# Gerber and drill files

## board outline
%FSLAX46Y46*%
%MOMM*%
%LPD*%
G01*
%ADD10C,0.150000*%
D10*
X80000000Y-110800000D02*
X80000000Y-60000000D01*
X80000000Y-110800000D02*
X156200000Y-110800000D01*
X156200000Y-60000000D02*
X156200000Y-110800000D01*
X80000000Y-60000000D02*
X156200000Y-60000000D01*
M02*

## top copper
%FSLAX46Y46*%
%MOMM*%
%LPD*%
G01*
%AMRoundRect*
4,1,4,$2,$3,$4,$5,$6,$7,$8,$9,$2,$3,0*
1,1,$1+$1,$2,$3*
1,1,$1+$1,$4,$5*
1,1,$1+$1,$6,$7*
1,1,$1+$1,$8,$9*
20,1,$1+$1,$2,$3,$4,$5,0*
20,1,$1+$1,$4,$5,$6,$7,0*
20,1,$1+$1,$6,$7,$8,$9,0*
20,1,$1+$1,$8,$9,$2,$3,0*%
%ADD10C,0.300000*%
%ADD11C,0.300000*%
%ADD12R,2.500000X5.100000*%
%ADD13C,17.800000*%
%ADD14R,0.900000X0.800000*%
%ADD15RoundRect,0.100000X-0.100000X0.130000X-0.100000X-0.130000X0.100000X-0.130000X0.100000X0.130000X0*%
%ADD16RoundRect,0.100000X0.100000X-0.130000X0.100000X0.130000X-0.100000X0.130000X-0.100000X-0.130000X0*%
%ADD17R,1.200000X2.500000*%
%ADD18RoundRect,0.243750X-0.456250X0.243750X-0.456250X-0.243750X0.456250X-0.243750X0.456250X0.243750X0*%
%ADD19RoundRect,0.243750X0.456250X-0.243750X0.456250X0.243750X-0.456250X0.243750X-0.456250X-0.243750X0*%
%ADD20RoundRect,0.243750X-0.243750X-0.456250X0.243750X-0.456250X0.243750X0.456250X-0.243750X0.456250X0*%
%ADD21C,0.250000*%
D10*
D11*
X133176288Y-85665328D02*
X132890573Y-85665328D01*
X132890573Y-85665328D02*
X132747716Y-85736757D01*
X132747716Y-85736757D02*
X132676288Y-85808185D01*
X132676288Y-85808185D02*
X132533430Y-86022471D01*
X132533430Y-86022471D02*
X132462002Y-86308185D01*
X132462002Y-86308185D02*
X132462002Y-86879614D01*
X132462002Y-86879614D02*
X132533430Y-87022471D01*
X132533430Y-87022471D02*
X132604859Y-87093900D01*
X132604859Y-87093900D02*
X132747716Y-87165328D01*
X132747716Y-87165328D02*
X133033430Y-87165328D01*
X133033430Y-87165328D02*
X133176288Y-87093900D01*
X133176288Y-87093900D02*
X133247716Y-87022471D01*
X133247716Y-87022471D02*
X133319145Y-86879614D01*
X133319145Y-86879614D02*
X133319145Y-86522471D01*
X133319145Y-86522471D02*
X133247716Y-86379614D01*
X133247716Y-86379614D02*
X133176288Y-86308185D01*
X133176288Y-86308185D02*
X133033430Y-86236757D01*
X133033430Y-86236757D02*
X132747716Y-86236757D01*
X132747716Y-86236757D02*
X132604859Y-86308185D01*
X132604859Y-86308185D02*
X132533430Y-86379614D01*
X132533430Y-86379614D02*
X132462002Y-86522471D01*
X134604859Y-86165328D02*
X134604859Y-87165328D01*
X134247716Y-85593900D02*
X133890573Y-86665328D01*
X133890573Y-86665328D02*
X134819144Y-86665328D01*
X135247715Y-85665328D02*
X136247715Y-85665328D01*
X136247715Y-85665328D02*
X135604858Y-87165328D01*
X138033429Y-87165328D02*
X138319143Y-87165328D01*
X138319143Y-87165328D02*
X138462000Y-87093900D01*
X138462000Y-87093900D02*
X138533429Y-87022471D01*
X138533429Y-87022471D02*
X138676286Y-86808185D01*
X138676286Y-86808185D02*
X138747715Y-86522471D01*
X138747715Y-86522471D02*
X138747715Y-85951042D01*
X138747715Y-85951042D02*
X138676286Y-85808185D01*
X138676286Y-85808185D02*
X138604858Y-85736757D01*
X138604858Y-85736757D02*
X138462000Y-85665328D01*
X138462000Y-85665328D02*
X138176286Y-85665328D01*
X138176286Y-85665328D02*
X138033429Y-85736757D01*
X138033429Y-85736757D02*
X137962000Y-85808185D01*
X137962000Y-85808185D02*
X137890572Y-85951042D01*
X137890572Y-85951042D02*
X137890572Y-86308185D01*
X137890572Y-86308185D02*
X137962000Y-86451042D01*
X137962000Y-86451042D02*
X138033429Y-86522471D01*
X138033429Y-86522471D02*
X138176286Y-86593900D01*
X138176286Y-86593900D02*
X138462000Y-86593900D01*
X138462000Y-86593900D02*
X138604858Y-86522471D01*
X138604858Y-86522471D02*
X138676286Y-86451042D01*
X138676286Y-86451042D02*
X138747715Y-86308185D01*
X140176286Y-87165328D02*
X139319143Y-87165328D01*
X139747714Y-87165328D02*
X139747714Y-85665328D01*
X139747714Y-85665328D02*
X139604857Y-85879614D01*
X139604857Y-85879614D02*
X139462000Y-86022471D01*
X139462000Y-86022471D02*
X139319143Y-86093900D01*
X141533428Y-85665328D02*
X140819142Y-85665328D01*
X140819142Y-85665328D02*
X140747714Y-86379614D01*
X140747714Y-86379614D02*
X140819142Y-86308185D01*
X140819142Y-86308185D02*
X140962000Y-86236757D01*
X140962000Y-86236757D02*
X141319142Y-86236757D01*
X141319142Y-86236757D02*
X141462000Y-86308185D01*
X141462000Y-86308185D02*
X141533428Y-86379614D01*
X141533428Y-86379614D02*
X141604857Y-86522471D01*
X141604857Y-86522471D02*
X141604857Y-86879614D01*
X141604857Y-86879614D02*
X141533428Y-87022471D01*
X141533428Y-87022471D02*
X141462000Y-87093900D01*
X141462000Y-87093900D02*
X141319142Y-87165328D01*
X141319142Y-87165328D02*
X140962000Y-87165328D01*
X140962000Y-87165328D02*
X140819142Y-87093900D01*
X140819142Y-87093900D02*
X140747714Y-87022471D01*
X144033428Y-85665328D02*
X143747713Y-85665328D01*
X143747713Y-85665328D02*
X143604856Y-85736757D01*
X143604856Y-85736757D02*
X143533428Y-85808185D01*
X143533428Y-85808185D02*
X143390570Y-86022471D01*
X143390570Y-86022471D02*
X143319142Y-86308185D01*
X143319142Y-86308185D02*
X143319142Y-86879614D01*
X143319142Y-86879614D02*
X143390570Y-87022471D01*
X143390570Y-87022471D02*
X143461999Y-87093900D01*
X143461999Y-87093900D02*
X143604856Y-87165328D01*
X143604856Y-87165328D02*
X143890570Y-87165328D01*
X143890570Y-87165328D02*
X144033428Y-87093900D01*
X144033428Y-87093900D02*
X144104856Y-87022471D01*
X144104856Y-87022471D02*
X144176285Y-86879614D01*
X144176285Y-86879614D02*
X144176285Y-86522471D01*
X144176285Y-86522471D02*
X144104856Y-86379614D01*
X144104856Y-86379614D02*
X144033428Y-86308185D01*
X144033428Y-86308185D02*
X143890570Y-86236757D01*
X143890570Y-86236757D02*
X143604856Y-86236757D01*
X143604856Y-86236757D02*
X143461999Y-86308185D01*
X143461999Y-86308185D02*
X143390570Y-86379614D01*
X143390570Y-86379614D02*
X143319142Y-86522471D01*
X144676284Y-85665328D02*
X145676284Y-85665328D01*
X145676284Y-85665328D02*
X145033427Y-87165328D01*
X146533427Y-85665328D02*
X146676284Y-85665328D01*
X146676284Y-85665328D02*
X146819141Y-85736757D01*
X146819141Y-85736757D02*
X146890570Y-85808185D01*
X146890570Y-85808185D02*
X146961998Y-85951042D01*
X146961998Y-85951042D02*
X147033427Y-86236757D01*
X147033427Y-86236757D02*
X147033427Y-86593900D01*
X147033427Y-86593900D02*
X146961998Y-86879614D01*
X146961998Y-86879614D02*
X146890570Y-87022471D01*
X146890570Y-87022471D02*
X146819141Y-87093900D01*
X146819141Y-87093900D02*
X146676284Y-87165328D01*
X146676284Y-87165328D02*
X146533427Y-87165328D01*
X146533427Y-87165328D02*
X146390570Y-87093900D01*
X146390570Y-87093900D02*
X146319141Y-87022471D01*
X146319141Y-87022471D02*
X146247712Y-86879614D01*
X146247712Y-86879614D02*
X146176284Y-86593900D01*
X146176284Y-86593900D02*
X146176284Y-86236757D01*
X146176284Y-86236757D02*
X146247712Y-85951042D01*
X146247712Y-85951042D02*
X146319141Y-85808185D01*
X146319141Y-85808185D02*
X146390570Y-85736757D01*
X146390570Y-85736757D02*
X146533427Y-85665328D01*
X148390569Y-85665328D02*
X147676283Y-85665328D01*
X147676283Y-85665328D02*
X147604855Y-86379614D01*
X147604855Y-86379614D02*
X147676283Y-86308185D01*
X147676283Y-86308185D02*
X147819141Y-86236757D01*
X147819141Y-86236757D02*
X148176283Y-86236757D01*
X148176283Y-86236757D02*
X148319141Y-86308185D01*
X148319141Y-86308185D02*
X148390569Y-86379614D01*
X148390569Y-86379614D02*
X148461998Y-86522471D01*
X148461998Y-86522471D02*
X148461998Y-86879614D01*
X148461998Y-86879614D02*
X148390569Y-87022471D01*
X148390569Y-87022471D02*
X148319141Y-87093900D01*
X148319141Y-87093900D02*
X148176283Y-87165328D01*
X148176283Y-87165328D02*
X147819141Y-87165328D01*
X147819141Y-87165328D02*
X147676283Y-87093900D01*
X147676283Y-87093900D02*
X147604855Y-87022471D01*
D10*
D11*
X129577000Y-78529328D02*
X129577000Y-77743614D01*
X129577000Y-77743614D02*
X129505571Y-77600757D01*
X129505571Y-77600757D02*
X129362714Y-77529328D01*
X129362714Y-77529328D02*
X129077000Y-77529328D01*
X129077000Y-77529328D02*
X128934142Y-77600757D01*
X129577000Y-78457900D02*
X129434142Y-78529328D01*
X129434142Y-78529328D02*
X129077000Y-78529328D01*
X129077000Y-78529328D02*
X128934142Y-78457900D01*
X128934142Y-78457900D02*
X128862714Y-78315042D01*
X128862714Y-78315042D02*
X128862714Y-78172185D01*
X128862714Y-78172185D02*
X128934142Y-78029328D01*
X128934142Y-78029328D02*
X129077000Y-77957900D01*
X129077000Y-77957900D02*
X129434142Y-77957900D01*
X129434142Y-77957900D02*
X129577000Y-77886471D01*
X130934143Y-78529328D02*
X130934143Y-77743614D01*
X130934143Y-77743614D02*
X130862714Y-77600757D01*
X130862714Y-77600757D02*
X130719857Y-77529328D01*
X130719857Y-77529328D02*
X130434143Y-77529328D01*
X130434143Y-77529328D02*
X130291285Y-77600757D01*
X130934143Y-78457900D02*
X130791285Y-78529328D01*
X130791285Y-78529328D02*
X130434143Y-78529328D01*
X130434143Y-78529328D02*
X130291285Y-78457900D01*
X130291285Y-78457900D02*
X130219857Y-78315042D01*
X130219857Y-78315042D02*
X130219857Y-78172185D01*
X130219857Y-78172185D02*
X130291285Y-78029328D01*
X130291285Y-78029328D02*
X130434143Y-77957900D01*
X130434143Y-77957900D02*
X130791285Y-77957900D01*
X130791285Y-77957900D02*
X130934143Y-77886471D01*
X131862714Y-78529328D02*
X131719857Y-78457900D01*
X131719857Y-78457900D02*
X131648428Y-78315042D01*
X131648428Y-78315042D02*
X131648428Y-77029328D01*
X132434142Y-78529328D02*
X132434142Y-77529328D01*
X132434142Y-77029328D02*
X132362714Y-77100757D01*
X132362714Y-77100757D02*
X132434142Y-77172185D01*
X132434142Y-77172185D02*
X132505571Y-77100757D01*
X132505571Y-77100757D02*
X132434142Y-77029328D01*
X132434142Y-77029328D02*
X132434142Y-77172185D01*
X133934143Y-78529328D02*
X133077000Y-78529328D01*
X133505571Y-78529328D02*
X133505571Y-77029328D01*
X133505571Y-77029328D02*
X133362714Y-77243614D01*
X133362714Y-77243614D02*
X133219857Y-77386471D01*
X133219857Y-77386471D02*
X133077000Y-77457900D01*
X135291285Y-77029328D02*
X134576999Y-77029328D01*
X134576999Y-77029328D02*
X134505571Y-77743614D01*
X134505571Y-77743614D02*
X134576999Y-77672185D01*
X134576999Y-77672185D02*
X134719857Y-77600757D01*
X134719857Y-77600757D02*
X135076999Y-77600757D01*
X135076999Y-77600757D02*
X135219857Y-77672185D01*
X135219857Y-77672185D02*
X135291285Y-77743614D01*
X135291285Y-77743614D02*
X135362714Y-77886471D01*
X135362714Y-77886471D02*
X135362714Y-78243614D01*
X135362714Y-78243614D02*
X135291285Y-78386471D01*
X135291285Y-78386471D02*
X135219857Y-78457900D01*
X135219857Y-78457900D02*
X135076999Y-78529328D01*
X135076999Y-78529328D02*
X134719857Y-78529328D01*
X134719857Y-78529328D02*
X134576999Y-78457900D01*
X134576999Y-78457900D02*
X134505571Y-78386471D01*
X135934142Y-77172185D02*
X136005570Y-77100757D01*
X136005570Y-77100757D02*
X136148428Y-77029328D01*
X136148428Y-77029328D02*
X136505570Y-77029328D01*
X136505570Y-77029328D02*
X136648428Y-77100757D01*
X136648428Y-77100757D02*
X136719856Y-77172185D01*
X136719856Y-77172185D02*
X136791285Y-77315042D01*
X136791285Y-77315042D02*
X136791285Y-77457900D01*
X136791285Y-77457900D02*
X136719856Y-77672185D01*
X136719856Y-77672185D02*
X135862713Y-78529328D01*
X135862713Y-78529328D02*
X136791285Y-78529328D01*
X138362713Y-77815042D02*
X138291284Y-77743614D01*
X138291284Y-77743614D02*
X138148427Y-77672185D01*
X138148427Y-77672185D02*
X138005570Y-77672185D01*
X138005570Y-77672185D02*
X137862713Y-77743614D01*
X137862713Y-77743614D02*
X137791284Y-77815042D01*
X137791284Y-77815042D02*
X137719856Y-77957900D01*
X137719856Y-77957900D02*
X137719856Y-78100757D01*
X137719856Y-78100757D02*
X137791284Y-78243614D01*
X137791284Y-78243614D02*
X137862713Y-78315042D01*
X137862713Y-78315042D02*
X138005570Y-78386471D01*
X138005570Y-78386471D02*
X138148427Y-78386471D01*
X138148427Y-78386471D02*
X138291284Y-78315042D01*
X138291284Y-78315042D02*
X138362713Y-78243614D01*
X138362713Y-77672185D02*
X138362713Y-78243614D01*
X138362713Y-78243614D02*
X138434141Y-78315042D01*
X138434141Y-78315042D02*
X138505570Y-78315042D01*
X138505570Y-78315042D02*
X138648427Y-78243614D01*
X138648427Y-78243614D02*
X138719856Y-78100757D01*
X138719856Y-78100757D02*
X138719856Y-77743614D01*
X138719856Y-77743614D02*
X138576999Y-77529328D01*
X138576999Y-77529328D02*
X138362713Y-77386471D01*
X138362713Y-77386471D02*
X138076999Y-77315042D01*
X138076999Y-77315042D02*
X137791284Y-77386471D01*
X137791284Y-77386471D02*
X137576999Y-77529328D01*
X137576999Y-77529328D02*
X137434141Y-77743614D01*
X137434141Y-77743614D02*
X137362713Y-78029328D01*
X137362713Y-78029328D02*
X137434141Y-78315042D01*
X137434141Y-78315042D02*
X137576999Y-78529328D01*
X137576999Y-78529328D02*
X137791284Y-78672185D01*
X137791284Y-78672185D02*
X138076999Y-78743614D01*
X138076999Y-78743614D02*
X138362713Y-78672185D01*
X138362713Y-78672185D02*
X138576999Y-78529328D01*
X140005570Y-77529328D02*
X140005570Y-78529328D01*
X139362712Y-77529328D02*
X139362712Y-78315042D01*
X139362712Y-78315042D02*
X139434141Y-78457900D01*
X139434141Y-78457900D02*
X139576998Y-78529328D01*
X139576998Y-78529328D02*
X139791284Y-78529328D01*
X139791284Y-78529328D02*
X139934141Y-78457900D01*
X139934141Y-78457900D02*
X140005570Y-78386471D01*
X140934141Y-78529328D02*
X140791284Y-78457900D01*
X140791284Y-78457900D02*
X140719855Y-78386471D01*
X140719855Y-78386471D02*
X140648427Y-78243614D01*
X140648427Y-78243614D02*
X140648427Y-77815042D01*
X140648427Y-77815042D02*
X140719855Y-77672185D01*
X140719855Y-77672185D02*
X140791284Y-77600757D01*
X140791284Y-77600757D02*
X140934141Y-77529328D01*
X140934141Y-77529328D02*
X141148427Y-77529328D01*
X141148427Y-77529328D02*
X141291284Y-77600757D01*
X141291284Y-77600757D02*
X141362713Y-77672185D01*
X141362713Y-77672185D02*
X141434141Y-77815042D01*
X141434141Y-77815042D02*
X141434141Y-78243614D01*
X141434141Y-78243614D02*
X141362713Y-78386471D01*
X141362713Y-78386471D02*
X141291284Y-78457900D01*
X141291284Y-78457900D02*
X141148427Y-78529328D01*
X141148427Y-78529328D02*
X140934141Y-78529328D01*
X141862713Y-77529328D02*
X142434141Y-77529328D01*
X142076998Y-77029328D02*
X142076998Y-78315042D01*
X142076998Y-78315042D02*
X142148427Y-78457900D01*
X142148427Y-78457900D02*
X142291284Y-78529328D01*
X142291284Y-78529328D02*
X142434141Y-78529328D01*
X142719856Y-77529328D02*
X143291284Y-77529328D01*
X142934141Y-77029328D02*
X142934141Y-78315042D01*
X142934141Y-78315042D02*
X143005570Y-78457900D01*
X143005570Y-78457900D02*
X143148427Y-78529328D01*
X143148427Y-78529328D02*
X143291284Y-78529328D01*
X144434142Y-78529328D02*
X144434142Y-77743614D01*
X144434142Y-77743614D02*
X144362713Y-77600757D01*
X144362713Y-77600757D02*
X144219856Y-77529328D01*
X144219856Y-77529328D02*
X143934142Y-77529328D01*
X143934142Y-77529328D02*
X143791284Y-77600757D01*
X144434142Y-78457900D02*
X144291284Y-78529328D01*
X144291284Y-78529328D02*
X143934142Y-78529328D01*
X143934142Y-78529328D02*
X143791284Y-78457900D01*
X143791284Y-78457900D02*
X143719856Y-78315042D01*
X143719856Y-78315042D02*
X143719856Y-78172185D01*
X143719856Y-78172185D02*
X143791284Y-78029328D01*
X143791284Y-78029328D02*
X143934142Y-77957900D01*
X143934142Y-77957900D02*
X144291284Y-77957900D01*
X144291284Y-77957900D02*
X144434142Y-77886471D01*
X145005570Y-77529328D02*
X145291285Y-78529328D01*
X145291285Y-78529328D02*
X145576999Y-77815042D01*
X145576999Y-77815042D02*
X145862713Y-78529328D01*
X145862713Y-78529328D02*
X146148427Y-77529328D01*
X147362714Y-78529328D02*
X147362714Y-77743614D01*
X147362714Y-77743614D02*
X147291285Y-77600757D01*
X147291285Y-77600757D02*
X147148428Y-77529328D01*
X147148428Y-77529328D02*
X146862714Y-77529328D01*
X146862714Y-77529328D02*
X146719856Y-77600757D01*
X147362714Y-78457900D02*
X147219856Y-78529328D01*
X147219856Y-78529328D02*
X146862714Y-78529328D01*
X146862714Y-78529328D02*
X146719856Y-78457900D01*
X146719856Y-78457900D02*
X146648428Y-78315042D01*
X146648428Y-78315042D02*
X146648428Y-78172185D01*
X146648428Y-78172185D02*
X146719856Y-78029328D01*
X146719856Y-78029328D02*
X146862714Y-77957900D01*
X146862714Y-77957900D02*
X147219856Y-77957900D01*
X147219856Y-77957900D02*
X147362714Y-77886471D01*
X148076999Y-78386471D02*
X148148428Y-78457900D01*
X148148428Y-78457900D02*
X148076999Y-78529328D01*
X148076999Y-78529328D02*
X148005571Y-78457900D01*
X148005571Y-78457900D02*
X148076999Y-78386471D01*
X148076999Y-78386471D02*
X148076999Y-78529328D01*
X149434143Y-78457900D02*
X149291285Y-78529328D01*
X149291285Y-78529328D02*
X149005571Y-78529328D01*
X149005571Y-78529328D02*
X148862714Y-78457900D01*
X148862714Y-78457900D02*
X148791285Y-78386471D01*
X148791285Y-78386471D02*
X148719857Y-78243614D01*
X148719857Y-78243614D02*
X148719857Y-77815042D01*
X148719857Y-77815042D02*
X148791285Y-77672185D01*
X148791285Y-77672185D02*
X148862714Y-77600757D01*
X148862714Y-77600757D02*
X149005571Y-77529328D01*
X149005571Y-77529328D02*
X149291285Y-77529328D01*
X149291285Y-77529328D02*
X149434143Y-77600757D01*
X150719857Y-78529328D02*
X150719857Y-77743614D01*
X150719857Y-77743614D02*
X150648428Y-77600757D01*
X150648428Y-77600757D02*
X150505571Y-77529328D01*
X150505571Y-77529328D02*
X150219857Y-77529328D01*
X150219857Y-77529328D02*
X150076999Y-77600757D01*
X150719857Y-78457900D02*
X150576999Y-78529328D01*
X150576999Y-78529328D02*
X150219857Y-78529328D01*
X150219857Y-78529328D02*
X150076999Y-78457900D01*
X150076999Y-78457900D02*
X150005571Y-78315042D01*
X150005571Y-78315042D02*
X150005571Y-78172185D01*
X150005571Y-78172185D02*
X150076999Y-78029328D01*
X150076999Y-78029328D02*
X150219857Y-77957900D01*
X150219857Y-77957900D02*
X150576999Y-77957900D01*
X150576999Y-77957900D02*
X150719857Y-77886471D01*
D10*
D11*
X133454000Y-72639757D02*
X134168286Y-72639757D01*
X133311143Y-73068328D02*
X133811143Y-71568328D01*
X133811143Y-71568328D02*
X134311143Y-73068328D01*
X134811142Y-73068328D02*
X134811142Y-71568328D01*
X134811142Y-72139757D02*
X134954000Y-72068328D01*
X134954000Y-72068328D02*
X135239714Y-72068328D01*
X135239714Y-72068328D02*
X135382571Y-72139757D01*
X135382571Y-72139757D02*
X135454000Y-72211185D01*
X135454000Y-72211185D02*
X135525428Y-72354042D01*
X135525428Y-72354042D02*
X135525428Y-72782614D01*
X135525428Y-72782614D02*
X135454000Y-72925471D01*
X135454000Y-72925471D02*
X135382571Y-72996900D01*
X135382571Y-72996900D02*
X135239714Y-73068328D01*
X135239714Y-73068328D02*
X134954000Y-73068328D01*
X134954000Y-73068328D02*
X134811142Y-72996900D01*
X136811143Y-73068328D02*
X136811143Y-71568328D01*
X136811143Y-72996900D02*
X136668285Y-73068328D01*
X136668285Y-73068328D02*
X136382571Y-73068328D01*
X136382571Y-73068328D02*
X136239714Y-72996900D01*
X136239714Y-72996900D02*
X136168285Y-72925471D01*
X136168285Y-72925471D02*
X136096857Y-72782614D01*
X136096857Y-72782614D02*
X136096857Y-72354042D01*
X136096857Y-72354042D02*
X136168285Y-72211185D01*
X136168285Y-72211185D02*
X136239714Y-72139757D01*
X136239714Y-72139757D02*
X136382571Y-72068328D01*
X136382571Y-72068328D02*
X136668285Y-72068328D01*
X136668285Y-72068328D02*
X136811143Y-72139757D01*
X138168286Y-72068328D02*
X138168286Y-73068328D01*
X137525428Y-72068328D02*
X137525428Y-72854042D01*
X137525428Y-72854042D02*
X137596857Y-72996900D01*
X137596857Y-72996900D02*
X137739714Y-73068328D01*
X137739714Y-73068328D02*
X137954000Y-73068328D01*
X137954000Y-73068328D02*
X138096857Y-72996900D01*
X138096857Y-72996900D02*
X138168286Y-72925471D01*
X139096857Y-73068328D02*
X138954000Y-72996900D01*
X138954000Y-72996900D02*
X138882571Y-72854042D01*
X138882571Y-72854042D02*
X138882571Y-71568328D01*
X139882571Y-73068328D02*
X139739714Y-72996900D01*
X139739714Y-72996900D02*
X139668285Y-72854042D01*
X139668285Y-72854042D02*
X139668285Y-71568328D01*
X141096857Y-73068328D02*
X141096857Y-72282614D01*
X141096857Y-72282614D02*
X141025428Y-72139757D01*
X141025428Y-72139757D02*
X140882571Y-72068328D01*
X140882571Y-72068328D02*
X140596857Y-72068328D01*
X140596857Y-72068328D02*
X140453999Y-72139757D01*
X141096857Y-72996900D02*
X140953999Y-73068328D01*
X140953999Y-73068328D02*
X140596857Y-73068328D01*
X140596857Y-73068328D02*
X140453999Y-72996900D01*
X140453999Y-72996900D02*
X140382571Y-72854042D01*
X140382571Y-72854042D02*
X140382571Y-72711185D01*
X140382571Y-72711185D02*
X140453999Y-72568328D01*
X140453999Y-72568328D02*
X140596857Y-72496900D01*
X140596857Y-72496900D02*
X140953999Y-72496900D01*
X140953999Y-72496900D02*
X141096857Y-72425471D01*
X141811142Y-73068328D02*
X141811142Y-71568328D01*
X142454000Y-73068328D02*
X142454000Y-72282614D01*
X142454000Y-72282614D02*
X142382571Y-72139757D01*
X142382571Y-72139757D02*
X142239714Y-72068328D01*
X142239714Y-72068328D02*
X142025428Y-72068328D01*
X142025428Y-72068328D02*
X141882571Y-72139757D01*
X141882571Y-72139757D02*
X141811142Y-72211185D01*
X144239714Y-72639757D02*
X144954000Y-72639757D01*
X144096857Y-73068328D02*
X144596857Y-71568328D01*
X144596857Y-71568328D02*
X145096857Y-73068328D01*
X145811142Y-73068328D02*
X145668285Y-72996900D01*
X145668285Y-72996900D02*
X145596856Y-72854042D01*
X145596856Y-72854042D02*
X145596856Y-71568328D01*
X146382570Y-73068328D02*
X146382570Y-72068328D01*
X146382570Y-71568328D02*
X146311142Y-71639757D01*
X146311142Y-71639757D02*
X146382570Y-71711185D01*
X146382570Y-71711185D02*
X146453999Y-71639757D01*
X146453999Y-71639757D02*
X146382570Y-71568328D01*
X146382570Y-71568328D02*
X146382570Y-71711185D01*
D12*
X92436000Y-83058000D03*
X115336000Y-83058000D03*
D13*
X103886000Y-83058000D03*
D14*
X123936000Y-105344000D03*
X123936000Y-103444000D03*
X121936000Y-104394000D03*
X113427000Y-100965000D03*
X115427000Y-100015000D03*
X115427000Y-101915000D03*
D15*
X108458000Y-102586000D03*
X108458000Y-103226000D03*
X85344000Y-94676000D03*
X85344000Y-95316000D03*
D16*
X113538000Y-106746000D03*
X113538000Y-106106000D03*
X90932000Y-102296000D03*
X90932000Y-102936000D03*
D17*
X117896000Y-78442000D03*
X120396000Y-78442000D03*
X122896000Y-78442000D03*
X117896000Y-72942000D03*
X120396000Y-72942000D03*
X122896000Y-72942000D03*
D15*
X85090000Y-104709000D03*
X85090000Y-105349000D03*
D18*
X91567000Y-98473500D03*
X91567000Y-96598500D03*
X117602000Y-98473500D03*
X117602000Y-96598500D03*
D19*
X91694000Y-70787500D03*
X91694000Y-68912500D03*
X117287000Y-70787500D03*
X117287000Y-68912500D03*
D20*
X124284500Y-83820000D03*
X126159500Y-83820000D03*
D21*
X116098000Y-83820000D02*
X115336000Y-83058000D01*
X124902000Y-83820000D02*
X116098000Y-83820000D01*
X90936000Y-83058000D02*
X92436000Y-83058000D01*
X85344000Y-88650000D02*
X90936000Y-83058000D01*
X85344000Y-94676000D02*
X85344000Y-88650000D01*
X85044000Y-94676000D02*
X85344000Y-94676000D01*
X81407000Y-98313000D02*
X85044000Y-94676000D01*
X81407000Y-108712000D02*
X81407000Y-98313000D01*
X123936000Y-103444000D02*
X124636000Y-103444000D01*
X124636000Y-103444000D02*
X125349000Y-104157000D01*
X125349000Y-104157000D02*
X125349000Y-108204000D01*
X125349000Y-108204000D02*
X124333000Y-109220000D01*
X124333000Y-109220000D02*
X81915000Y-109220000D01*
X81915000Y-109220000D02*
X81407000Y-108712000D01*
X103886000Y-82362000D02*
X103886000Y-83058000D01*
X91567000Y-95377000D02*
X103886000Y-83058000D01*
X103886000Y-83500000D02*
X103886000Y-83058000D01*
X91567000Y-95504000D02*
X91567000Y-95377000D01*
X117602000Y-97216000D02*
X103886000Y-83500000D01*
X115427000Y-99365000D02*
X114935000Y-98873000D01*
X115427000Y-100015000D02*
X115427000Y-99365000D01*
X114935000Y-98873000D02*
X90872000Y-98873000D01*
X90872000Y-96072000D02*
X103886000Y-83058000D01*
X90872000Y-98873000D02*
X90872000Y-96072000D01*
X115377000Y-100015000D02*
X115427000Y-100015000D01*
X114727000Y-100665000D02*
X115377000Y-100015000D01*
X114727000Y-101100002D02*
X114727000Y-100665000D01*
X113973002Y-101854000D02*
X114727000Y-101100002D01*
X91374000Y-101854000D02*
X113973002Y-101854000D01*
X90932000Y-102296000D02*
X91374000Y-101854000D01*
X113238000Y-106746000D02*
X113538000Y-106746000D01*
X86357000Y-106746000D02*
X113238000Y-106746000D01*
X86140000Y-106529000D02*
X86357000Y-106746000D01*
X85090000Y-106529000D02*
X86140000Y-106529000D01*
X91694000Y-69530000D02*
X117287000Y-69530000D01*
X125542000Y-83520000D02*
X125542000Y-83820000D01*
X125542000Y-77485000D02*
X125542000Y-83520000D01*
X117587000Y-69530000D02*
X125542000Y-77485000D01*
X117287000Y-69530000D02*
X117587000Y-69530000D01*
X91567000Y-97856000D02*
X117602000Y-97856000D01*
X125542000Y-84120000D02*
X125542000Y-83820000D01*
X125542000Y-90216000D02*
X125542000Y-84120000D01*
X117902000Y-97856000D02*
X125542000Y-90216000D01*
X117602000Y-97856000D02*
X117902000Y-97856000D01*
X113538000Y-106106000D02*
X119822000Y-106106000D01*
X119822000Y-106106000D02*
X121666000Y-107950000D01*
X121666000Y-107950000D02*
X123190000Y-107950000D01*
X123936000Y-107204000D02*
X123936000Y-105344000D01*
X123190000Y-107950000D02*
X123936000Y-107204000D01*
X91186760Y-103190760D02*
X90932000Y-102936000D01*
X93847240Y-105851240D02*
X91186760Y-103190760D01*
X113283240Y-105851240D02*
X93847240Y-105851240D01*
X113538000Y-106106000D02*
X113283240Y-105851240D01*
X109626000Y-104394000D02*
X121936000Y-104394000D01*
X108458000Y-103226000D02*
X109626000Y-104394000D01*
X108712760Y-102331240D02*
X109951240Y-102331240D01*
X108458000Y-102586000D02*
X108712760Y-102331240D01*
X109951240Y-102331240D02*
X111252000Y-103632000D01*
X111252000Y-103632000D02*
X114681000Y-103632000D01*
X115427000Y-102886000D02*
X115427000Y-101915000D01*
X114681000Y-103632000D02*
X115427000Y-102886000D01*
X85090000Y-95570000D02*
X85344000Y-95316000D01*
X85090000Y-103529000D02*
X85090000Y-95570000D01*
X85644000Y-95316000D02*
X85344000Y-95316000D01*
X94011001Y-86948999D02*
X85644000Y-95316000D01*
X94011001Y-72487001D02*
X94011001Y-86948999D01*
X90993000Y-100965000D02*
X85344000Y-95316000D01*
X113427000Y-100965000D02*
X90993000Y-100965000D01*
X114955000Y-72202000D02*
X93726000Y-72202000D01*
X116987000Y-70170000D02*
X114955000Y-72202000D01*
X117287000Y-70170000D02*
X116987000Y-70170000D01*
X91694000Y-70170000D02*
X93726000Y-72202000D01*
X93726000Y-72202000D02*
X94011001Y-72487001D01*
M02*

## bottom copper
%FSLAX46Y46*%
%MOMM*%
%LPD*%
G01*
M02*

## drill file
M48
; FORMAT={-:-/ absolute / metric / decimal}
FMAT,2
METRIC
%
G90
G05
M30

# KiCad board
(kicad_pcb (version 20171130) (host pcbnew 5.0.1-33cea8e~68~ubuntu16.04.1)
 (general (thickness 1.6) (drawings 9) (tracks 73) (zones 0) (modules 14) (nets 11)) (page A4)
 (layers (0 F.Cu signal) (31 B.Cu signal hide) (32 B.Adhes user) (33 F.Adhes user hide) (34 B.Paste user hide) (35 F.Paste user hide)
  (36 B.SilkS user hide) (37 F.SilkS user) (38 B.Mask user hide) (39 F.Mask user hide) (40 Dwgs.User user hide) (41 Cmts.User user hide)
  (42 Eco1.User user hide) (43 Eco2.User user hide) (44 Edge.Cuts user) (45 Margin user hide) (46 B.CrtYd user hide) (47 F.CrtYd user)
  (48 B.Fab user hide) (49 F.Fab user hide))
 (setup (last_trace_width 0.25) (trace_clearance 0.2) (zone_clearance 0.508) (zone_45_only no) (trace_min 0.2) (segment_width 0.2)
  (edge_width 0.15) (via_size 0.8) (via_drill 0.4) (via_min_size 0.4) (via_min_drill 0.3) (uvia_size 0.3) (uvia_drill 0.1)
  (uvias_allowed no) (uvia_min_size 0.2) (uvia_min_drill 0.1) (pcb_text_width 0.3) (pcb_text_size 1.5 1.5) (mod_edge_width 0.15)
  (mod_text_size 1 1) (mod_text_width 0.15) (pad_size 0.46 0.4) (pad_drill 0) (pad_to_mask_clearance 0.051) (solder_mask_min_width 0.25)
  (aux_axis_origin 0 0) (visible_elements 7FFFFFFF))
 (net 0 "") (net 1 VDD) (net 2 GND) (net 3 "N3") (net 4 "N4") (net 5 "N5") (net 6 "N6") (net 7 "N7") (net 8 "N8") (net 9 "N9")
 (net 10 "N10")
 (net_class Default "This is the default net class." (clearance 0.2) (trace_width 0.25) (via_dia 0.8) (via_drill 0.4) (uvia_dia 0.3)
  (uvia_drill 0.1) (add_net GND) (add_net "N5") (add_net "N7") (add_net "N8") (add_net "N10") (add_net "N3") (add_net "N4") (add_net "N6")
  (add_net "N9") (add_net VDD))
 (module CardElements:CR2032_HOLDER (layer F.Cu) (at 103.886 83.058)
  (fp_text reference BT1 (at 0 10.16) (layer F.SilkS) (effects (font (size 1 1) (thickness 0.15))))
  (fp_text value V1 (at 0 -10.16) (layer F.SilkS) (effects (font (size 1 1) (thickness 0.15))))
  (pad 1 smd rect (at -11.45 0) (size 2.5 5.1) (layers F.Cu F.Paste F.Mask) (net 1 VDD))
  (pad 1 smd rect (at 11.45 0) (size 2.5 5.1) (layers F.Cu F.Paste F.Mask) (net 1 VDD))
  (pad 2 smd circle (at 0 0) (size 17.8 17.8) (layers F.Cu F.Paste F.Mask) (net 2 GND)))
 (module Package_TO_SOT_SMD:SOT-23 (layer F.Cu) (at 122.936 104.394 180)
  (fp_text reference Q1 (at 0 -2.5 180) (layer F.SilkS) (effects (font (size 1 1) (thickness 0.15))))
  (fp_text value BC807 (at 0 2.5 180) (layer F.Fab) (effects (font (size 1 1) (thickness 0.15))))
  (pad 1 smd rect (at -1 -0.95 180) (size 0.9 0.8) (layers F.Cu F.Paste F.Mask) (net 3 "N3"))
  (pad 2 smd rect (at -1 0.95 180) (size 0.9 0.8) (layers F.Cu F.Paste F.Mask) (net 1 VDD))
  (pad 3 smd rect (at 1 0 180) (size 0.9 0.8) (layers F.Cu F.Paste F.Mask) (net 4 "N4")))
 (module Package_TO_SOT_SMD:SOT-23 (layer F.Cu) (at 114.427 100.965 180)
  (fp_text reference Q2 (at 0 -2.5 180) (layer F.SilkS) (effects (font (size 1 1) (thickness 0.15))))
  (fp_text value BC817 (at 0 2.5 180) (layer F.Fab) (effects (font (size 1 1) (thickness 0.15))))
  (pad 3 smd rect (at 1 0 180) (size 0.9 0.8) (layers F.Cu F.Paste F.Mask) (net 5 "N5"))
  (pad 2 smd rect (at -1 0.95 180) (size 0.9 0.8) (layers F.Cu F.Paste F.Mask) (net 2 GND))
  (pad 1 smd rect (at -1 -0.95 180) (size 0.9 0.8) (layers F.Cu F.Paste F.Mask) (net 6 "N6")))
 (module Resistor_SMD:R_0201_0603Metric (layer F.Cu) (at 108.458 102.906 270)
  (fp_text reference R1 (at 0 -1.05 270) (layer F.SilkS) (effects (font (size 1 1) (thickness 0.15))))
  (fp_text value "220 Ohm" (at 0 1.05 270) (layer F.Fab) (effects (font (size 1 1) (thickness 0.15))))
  (pad "" smd roundrect (at -0.345 0 270) (size 0.318 0.36) (layers F.Paste) (roundrect_rratio 0.25))
  (pad "" smd roundrect (at 0.345 0 270) (size 0.318 0.36) (layers F.Paste) (roundrect_rratio 0.25))
  (pad 1 smd roundrect (at -0.32 0 270) (size 0.46 0.4) (layers F.Cu F.Mask) (roundrect_rratio 0.25) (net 6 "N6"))
  (pad 2 smd roundrect (at 0.32 0 270) (size 0.46 0.4) (layers F.Cu F.Mask) (roundrect_rratio 0.25) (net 4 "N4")))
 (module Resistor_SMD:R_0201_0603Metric (layer F.Cu) (at 85.344 94.996 270)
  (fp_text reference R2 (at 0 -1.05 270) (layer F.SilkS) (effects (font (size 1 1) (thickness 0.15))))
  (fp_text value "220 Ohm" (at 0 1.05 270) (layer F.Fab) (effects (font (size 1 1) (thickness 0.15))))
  (pad "" smd roundrect (at -0.345 0 270) (size 0.318 0.36) (layers F.Paste) (roundrect_rratio 0.25))
  (pad "" smd roundrect (at 0.345 0 270) (size 0.318 0.36) (layers F.Paste) (roundrect_rratio 0.25))
  (pad 1 smd roundrect (at -0.32 0 270) (size 0.46 0.4) (layers F.Cu F.Mask) (roundrect_rratio 0.25) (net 1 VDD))
  (pad 2 smd roundrect (at 0.32 0 270) (size 0.46 0.4) (layers F.Cu F.Mask) (roundrect_rratio 0.25) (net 5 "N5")))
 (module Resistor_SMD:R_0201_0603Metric (layer F.Cu) (at 113.538 106.426 90)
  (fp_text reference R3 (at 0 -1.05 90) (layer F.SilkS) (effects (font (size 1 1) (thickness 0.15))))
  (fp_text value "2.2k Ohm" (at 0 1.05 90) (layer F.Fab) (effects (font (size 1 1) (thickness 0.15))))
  (pad "" smd roundrect (at -0.345 0 90) (size 0.318 0.36) (layers F.Paste) (roundrect_rratio 0.25))
  (pad "" smd roundrect (at 0.345 0 90) (size 0.318 0.36) (layers F.Paste) (roundrect_rratio 0.25))
  (pad 1 smd roundrect (at -0.32 0 90) (size 0.46 0.4) (layers F.Cu F.Mask) (roundrect_rratio 0.25) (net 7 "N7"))
  (pad 2 smd roundrect (at 0.32 0 90) (size 0.46 0.4) (layers F.Cu F.Mask) (roundrect_rratio 0.25) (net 3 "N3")))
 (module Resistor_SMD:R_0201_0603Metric (layer F.Cu) (at 90.932 102.616 90)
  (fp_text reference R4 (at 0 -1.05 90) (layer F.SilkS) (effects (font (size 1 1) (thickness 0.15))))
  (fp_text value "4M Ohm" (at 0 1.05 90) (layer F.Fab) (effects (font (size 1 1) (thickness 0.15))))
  (pad 2 smd roundrect (at 0.32 0 90) (size 0.46 0.4) (layers F.Cu F.Mask) (roundrect_rratio 0.25) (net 2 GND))
  (pad 1 smd roundrect (at -0.32 0 90) (size 0.46 0.4) (layers F.Cu F.Mask) (roundrect_rratio 0.25) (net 3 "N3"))
  (pad "" smd roundrect (at 0.345 0 90) (size 0.318 0.36) (layers F.Paste) (roundrect_rratio 0.25))
  (pad "" smd roundrect (at -0.345 0 90) (size 0.318 0.36) (layers F.Paste) (roundrect_rratio 0.25)))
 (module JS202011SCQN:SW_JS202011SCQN (layer F.Cu) (at 120.396 75.692)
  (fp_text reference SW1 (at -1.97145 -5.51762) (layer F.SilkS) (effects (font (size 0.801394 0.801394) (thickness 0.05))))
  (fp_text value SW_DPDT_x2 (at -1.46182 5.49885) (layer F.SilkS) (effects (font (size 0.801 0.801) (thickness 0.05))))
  (pad 1 smd rect (at -2.5 2.75) (size 1.2 2.5) (layers F.Cu F.Paste F.Mask) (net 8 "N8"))
  (pad 2 smd rect (at 0 2.75) (size 1.2 2.5) (layers F.Cu F.Paste F.Mask) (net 5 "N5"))
  (pad 3 smd rect (at 2.5 2.75) (size 1.2 2.5) (layers F.Cu F.Paste F.Mask) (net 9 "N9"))
  (pad 4 smd rect (at -2.5 -2.75) (size 1.2 2.5) (layers F.Cu F.Paste F.Mask))
  (pad 5 smd rect (at 0 -2.75) (size 1.2 2.5) (layers F.Cu F.Paste F.Mask))
  (pad 6 smd rect (at 2.5 -2.75) (size 1.2 2.5) (layers F.Cu F.Paste F.Mask)))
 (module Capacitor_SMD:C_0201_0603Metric (layer F.Cu) (at 85.09 105.029 270)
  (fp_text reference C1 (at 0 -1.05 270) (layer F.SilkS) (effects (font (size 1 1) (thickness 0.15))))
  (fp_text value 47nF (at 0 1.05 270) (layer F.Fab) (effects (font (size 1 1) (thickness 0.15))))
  (pad "" smd roundrect (at -0.345 0 270) (size 0.318 0.36) (layers F.Paste) (roundrect_rratio 0.25))
  (pad "" smd roundrect (at 0.345 0 270) (size 0.318 0.36) (layers F.Paste) (roundrect_rratio 0.25))
  (pad 1 smd roundrect (at -0.32 0 270) (size 0.46 0.4) (layers F.Cu F.Mask) (roundrect_rratio 0.25) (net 5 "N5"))
  (pad 2 smd roundrect (at 0.32 0 270) (size 0.46 0.4) (layers F.Cu F.Mask) (roundrect_rratio 0.25) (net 7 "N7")))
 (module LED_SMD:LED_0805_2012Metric (layer F.Cu) (at 91.567 97.536 270)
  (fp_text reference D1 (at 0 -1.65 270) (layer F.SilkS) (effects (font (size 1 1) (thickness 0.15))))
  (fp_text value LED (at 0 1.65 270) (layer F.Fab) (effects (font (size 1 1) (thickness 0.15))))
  (pad 2 smd roundrect (at 0.9375 0 270) (size 0.975 1.4) (layers F.Cu F.Paste F.Mask) (roundrect_rratio 0.25) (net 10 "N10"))
  (pad 1 smd roundrect (at -0.9375 0 270) (size 0.975 1.4) (layers F.Cu F.Paste F.Mask) (roundrect_rratio 0.25) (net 8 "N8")))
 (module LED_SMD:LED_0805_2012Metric (layer F.Cu) (at 117.602 97.536 270)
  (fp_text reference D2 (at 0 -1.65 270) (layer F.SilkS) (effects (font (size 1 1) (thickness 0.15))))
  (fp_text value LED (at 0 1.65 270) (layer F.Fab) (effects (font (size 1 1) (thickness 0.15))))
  (pad 2 smd roundrect (at 0.9375 0 270) (size 0.975 1.4) (layers F.Cu F.Paste F.Mask) (roundrect_rratio 0.25) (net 10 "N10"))
  (pad 1 smd roundrect (at -0.9375 0 270) (size 0.975 1.4) (layers F.Cu F.Paste F.Mask) (roundrect_rratio 0.25) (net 8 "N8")))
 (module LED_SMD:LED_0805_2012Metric (layer F.Cu) (at 91.694 69.85 90)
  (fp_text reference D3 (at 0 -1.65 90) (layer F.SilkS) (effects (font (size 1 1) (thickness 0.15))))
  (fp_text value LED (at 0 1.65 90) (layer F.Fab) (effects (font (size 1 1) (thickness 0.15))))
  (pad 1 smd roundrect (at -0.9375 0 90) (size 0.975 1.4) (layers F.Cu F.Paste F.Mask) (roundrect_rratio 0.25) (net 8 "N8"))
  (pad 2 smd roundrect (at 0.9375 0 90) (size 0.975 1.4) (layers F.Cu F.Paste F.Mask) (roundrect_rratio 0.25) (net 10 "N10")))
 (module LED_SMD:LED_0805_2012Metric (layer F.Cu) (at 117.287 69.85 90)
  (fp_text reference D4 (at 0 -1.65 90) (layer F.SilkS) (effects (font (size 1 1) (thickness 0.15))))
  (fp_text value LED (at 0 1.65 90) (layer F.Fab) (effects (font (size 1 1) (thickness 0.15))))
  (pad 1 smd roundrect (at -0.9375 0 90) (size 0.975 1.4) (layers F.Cu F.Paste F.Mask) (roundrect_rratio 0.25) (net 8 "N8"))
  (pad 2 smd roundrect (at 0.9375 0 90) (size 0.975 1.4) (layers F.Cu F.Paste F.Mask) (roundrect_rratio 0.25) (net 10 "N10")))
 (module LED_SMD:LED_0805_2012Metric (layer F.Cu) (at 125.222 83.82)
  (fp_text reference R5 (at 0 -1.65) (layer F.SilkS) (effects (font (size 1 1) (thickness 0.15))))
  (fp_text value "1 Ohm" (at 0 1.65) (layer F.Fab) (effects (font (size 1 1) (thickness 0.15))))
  (pad 1 smd roundrect (at -0.9375 0) (size 0.975 1.4) (layers F.Cu F.Paste F.Mask) (roundrect_rratio 0.25) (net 1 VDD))
  (pad 2 smd roundrect (at 0.9375 0) (size 0.975 1.4) (layers F.Cu F.Paste F.Mask) (roundrect_rratio 0.25) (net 10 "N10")))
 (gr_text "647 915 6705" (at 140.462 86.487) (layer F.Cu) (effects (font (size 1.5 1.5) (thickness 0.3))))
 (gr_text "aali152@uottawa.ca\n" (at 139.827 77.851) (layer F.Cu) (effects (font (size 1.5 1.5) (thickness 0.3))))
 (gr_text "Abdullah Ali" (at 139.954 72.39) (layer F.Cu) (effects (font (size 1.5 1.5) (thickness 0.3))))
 (gr_line (start 80 110.8) (end 80 60) (layer Edge.Cuts) (width 0.15))
 (gr_line (start 80 110.8) (end 156.2 110.8) (layer Edge.Cuts) (width 0.15))
 (gr_line (start 156.2 60) (end 156.2 110.8) (layer Edge.Cuts) (width 0.15))
 (gr_line (start 80 60) (end 156.2 60) (layer Edge.Cuts) (width 0.15))
 (segment (start 116.098 83.82) (end 115.336 83.058) (width 0.25) (layer F.Cu) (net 1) (status 30))
 (segment (start 124.902 83.82) (end 116.098 83.82) (width 0.25) (layer F.Cu) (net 1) (status 20))
 (segment (start 90.936 83.058) (end 92.436 83.058) (width 0.25) (layer F.Cu) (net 1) (status 20))
 (segment (start 85.344 88.65) (end 90.936 83.058) (width 0.25) (layer F.Cu) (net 1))
 (segment (start 85.344 94.676) (end 85.344 88.65) (width 0.25) (layer F.Cu) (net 1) (status 10))
 (segment (start 85.044 94.676) (end 85.344 94.676) (width 0.25) (layer F.Cu) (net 1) (status 20))
 (segment (start 81.407 98.313) (end 85.044 94.676) (width 0.25) (layer F.Cu) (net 1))
 (segment (start 81.407 108.712) (end 81.407 98.313) (width 0.25) (layer F.Cu) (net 1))
 (segment (start 123.936 103.444) (end 124.636 103.444) (width 0.25) (layer F.Cu) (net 1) (status 10))
 (segment (start 124.636 103.444) (end 125.349 104.157) (width 0.25) (layer F.Cu) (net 1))
 (segment (start 125.349 104.157) (end 125.349 108.204) (width 0.25) (layer F.Cu) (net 1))
 (segment (start 125.349 108.204) (end 124.333 109.22) (width 0.25) (layer F.Cu) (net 1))
 (segment (start 124.333 109.22) (end 81.915 109.22) (width 0.25) (layer F.Cu) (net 1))
 (segment (start 81.915 109.22) (end 81.407 108.712) (width 0.25) (layer F.Cu) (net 1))
 (segment (start 103.886 82.362) (end 103.886 83.058) (width 0.25) (layer F.Cu) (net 2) (status 30))
 (segment (start 91.567 95.377) (end 103.886 83.058) (width 0.25) (layer F.Cu) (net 2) (status 20))
 (segment (start 103.886 83.5) (end 103.886 83.058) (width 0.25) (layer F.Cu) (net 2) (status 30))
 (segment (start 91.567 95.504) (end 91.567 95.377) (width 0.25) (layer F.Cu) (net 2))
 (segment (start 117.602 97.216) (end 103.886 83.5) (width 0.25) (layer F.Cu) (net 2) (status 20))
 (segment (start 115.427 99.365) (end 114.935 98.873) (width 0.25) (layer F.Cu) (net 2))
 (segment (start 115.427 100.015) (end 115.427 99.365) (width 0.25) (layer F.Cu) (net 2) (status 10))
 (segment (start 114.935 98.873) (end 90.872 98.873) (width 0.25) (layer F.Cu) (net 2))
 (segment (start 90.872 96.072) (end 103.886 83.058) (width 0.25) (layer F.Cu) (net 2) (status 20))
 (segment (start 90.872 98.873) (end 90.872 96.072) (width 0.25) (layer F.Cu) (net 2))
 (segment (start 115.377 100.015) (end 115.427 100.015) (width 0.25) (layer F.Cu) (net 2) (status 30))
 (segment (start 114.727 100.665) (end 115.377 100.015) (width 0.25) (layer F.Cu) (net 2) (status 20))
 (segment (start 114.727 101.100002) (end 114.727 100.665) (width 0.25) (layer F.Cu) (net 2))
 (segment (start 113.973002 101.854) (end 114.727 101.100002) (width 0.25) (layer F.Cu) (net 2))
 (segment (start 91.374 101.854) (end 113.973002 101.854) (width 0.25) (layer F.Cu) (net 2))
 (segment (start 90.932 102.296) (end 91.374 101.854) (width 0.25) (layer F.Cu) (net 2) (status 10))
 (segment (start 113.238 106.746) (end 113.538 106.746) (width 0.25) (layer F.Cu) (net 7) (status 20))
 (segment (start 86.357 106.746) (end 113.238 106.746) (width 0.25) (layer F.Cu) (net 7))
 (segment (start 86.14 106.529) (end 86.357 106.746) (width 0.25) (layer F.Cu) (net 7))
 (segment (start 85.09 106.529) (end 86.14 106.529) (width 0.25) (layer F.Cu) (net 7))
 (segment (start 91.694 69.53) (end 117.287 69.53) (width 0.25) (layer F.Cu) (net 10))
 (segment (start 125.542 83.52) (end 125.542 83.82) (width 0.25) (layer F.Cu) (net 10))
 (segment (start 125.542 77.485) (end 125.542 83.52) (width 0.25) (layer F.Cu) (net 10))
 (segment (start 117.587 69.53) (end 125.542 77.485) (width 0.25) (layer F.Cu) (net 10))
 (segment (start 117.287 69.53) (end 117.587 69.53) (width 0.25) (layer F.Cu) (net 10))
 (segment (start 91.567 97.856) (end 117.602 97.856) (width 0.25) (layer F.Cu) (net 10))
 (segment (start 125.542 84.12) (end 125.542 83.82) (width 0.25) (layer F.Cu) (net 10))
 (segment (start 125.542 90.216) (end 125.542 84.12) (width 0.25) (layer F.Cu) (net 10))
 (segment (start 117.902 97.856) (end 125.542 90.216) (width 0.25) (layer F.Cu) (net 10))
 (segment (start 117.602 97.856) (end 117.902 97.856) (width 0.25) (layer F.Cu) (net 10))
 (segment (start 113.538 106.106) (end 119.822 106.106) (width 0.25) (layer F.Cu) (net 3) (status 10))
 (segment (start 119.822 106.106) (end 121.666 107.95) (width 0.25) (layer F.Cu) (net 3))
 (segment (start 121.666 107.95) (end 123.19 107.95) (width 0.25) (layer F.Cu) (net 3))
 (segment (start 123.936 107.204) (end 123.936 105.344) (width 0.25) (layer F.Cu) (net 3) (status 20))
 (segment (start 123.19 107.95) (end 123.936 107.204) (width 0.25) (layer F.Cu) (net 3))
 (segment (start 91.18676 103.19076) (end 90.932 102.936) (width 0.25) (layer F.Cu) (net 3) (status 20))
 (segment (start 93.84724 105.85124) (end 91.18676 103.19076) (width 0.25) (layer F.Cu) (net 3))
 (segment (start 113.28324 105.85124) (end 93.84724 105.85124) (width 0.25) (layer F.Cu) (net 3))
 (segment (start 113.538 106.106) (end 113.28324 105.85124) (width 0.25) (layer F.Cu) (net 3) (status 10))
 (segment (start 109.626 104.394) (end 121.936 104.394) (width 0.25) (layer F.Cu) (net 4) (status 20))
 (segment (start 108.458 103.226) (end 109.626 104.394) (width 0.25) (layer F.Cu) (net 4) (status 10))
 (segment (start 108.71276 102.33124) (end 109.95124 102.33124) (width 0.25) (layer F.Cu) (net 6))
 (segment (start 108.458 102.586) (end 108.71276 102.33124) (width 0.25) (layer F.Cu) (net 6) (status 10))
 (segment (start 109.95124 102.33124) (end 111.252 103.632) (width 0.25) (layer F.Cu) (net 6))
 (segment (start 111.252 103.632) (end 114.681 103.632) (width 0.25) (layer F.Cu) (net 6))
 (segment (start 115.427 102.886) (end 115.427 101.915) (width 0.25) (layer F.Cu) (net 6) (status 20))
 (segment (start 114.681 103.632) (end 115.427 102.886) (width 0.25) (layer F.Cu) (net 6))
 (segment (start 85.09 95.57) (end 85.344 95.316) (width 0.25) (layer F.Cu) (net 5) (status 20))
 (segment (start 85.09 103.529) (end 85.09 95.57) (width 0.25) (layer F.Cu) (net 5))
 (segment (start 85.644 95.316) (end 85.344 95.316) (width 0.25) (layer F.Cu) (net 5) (status 20))
 (segment (start 94.011001 86.948999) (end 85.644 95.316) (width 0.25) (layer F.Cu) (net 5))
 (segment (start 94.011001 72.487001) (end 94.011001 86.948999) (width 0.25) (layer F.Cu) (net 5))
 (segment (start 90.993 100.965) (end 85.344 95.316) (width 0.25) (layer F.Cu) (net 5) (status 20))
 (segment (start 113.427 100.965) (end 90.993 100.965) (width 0.25) (layer F.Cu) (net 5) (status 10))
 (segment (start 114.955 72.202) (end 93.726 72.202) (width 0.25) (layer F.Cu) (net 5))
 (segment (start 116.987 70.17) (end 114.955 72.202) (width 0.25) (layer F.Cu) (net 5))
 (segment (start 117.287 70.17) (end 116.987 70.17) (width 0.25) (layer F.Cu) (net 5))
 (segment (start 91.694 70.17) (end 93.726 72.202) (width 0.25) (layer F.Cu) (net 5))
 (segment (start 93.726 72.202) (end 94.011001 72.487001) (width 0.25) (layer F.Cu) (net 5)))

